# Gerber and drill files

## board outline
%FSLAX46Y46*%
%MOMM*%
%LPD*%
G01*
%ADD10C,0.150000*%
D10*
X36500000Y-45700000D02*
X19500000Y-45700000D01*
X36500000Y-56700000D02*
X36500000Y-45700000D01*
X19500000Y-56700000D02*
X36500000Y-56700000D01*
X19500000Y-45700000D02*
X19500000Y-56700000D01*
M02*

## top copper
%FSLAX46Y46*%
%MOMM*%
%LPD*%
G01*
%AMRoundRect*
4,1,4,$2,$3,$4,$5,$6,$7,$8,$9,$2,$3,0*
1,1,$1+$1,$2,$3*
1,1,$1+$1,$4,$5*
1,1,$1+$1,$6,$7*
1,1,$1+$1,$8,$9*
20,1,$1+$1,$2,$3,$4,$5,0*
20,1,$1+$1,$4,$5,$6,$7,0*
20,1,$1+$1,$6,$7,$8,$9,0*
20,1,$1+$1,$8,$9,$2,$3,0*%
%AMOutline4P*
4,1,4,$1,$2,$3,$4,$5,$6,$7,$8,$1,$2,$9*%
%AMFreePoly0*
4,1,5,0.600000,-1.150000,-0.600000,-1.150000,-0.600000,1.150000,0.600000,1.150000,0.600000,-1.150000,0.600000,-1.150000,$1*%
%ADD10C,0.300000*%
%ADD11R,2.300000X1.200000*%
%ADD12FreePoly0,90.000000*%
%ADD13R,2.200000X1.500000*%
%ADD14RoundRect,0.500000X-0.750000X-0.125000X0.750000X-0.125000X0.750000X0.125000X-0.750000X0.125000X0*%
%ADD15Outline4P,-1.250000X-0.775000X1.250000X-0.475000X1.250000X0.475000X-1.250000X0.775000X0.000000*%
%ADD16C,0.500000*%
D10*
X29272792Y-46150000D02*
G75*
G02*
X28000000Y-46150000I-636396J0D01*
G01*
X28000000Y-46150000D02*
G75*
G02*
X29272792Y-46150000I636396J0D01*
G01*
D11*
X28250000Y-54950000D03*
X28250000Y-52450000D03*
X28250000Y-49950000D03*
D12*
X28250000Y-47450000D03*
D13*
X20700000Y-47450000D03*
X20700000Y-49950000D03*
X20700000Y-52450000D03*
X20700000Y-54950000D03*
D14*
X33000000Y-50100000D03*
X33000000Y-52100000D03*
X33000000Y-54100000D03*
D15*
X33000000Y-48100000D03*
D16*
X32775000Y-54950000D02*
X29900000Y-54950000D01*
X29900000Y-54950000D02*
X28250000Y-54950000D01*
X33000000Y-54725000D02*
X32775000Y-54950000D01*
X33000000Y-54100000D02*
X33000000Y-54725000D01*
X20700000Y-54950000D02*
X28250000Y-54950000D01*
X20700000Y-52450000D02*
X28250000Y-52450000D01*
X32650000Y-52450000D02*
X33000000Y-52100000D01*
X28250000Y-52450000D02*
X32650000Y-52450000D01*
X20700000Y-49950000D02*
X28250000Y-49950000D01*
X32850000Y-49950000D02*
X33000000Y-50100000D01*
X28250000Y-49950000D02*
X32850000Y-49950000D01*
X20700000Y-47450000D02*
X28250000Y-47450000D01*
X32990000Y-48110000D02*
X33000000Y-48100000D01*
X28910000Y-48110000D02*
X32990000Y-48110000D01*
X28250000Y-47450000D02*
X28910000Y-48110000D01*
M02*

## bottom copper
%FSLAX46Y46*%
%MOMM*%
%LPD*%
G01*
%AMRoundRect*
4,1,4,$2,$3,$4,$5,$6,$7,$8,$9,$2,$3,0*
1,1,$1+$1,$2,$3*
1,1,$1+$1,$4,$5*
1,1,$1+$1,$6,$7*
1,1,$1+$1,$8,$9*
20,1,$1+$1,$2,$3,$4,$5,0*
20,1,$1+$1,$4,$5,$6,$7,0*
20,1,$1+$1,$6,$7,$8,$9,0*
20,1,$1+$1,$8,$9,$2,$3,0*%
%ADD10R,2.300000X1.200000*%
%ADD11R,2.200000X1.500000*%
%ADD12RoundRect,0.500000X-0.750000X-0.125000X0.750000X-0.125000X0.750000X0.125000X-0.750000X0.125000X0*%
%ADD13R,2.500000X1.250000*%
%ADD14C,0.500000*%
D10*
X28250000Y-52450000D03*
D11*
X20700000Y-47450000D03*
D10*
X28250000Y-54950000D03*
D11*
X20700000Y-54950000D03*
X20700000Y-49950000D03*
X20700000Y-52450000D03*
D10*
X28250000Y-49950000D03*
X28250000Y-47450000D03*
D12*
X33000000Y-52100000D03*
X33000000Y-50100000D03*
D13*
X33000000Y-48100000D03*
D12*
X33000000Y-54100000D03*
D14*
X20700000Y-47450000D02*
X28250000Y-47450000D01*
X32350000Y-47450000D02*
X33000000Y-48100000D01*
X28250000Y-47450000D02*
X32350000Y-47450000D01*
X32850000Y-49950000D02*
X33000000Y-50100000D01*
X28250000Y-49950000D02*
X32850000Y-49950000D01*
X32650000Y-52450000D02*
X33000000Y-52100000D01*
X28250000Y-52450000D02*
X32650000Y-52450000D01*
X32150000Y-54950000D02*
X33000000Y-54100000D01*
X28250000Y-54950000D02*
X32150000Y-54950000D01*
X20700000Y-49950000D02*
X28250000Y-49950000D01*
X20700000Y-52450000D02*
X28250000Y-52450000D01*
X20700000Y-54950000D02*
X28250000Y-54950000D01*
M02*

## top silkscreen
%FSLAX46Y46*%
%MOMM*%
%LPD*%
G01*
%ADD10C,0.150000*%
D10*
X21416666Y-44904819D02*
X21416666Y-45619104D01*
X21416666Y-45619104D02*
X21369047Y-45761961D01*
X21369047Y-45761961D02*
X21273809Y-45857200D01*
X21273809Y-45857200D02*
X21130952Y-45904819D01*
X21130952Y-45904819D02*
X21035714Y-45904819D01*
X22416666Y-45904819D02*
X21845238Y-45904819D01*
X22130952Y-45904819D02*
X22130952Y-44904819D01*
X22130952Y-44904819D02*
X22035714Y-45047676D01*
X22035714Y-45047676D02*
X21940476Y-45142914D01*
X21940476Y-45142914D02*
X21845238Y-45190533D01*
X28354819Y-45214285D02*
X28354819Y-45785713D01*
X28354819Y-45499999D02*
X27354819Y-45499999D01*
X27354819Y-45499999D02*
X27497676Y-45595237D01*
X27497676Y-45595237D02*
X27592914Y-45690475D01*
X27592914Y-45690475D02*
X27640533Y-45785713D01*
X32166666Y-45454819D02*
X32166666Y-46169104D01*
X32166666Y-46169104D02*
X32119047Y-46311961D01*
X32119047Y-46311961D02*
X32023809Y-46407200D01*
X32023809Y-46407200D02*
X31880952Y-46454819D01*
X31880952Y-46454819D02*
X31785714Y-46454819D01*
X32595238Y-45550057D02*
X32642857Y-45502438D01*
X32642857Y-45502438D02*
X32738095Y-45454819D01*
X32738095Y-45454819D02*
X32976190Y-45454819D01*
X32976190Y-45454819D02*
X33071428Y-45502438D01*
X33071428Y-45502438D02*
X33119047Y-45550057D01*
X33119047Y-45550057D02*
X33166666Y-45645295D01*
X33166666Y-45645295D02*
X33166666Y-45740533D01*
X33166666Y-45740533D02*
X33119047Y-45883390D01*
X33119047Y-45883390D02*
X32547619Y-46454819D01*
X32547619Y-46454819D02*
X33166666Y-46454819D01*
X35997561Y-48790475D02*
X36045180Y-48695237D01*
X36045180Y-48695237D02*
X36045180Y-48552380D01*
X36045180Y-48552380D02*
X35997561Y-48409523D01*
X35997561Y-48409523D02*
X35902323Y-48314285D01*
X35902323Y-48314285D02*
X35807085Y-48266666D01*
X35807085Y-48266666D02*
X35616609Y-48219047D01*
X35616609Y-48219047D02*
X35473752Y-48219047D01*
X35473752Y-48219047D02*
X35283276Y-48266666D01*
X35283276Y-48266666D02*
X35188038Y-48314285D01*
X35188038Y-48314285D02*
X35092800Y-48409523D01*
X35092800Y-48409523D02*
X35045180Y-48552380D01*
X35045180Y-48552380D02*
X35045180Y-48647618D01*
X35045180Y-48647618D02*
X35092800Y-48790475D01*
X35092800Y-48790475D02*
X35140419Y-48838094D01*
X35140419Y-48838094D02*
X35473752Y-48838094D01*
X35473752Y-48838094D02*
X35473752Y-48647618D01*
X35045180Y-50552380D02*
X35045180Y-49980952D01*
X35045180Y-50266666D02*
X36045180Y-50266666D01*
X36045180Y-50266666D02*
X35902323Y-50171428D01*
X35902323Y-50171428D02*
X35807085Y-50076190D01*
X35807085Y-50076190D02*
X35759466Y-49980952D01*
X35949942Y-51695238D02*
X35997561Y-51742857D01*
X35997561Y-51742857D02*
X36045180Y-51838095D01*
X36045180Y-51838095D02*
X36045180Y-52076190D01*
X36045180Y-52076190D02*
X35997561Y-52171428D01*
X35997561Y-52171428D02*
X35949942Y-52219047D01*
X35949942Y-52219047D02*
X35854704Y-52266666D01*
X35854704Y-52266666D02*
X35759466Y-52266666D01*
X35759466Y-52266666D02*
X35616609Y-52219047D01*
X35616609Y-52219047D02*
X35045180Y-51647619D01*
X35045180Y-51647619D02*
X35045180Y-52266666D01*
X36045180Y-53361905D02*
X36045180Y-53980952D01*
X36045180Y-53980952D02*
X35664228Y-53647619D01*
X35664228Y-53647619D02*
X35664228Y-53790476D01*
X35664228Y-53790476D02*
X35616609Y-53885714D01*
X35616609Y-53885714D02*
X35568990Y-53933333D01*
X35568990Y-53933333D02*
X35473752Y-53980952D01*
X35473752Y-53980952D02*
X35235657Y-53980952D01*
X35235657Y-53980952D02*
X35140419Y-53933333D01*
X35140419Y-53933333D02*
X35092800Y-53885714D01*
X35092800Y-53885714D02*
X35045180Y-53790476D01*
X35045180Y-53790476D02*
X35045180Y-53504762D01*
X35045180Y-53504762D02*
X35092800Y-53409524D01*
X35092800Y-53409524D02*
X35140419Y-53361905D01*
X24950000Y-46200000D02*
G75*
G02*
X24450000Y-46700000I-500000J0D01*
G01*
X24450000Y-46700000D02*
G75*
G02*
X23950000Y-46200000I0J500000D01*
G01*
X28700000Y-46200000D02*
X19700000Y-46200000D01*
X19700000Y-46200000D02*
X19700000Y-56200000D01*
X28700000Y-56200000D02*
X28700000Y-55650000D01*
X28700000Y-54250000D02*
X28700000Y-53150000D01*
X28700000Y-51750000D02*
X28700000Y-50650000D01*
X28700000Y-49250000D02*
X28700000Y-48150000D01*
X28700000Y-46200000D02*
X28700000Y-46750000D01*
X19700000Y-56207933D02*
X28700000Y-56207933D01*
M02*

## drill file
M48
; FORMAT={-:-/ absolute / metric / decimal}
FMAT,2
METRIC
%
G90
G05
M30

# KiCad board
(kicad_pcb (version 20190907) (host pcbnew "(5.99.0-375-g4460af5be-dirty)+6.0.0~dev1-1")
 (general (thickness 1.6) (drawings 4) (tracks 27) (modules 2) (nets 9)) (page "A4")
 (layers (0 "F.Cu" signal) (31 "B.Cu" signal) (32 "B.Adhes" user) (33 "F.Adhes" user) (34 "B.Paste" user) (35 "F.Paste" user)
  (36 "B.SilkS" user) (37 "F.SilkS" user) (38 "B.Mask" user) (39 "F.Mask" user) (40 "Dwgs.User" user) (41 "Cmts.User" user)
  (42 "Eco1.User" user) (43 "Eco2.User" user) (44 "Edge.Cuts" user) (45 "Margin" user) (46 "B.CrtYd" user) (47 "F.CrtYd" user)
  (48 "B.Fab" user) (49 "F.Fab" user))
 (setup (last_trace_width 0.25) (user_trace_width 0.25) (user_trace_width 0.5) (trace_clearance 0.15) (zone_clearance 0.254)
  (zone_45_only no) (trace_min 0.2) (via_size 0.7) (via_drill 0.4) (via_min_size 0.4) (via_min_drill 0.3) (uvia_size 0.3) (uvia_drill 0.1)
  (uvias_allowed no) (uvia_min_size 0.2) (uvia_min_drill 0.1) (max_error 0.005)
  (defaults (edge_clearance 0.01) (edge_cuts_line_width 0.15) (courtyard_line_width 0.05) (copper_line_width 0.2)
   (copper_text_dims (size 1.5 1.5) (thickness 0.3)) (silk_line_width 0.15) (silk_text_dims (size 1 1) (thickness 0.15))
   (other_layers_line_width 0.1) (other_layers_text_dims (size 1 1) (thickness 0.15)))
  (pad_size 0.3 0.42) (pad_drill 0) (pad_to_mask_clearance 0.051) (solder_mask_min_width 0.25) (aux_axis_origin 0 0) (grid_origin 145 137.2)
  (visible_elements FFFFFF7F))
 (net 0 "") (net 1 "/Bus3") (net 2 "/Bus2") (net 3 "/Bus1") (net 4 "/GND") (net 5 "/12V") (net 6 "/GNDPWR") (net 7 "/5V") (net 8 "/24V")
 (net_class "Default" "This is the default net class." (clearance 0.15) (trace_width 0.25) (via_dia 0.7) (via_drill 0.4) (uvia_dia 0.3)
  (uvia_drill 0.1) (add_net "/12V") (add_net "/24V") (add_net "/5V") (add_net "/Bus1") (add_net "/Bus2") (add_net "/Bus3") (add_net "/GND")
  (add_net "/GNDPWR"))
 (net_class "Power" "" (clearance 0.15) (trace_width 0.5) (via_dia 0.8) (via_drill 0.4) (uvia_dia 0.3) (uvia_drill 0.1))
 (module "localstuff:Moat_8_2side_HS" (layer "F.Cu") (at 24.5 56.2 -90)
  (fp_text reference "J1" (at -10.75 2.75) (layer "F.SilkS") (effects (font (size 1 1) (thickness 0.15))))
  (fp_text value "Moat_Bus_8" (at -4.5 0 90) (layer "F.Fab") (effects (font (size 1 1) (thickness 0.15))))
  (fp_arc (start -10 0.05) (end -10 -0.45) (angle 90) (layer "F.SilkS") (width 0.15))
  (fp_arc (start -10 0.05) (end -9.5 0.05) (angle 90) (layer "F.SilkS") (width 0.15))
  (fp_line (start -10 -4.2) (end -10 4.8) (layer "F.SilkS") (width 0.15))
  (fp_line (start -10 4.8) (end 0 4.8) (layer "F.SilkS") (width 0.15))
  (fp_line (start 0 -4.2) (end -0.55 -4.2) (layer "F.SilkS") (width 0.15))
  (fp_line (start -1.95 -4.2) (end -3.05 -4.2) (layer "F.SilkS") (width 0.15))
  (fp_line (start -4.45 -4.2) (end -5.55 -4.2) (layer "F.SilkS") (width 0.15))
  (fp_line (start -6.95 -4.2) (end -8.05 -4.2) (layer "F.SilkS") (width 0.15))
  (fp_line (start -10 -4.2) (end -9.45 -4.2) (layer "F.SilkS") (width 0.15))
  (fp_line (start 0.007933 4.8) (end 0.007933 -4.2) (layer "F.SilkS") (width 0.15))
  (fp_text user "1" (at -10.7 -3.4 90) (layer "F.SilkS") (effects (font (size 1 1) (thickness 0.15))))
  (fp_circle (center -10.05 -4.136396) (end -9.413604 -4.136396) (layer "F.Cu") (width 0.3))
  (pad "4" smd rect (at -1.25 -3.75 270) (size 1.2 2.3) (layers "F.Cu" "F.Paste" "F.Mask") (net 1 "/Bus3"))
  (pad "3" smd rect (at -3.75 -3.75 270) (size 1.2 2.3) (layers "F.Cu" "F.Paste" "F.Mask") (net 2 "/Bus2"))
  (pad "2" smd rect (at -6.25 -3.75 270) (size 1.2 2.3) (layers "F.Cu" "F.Paste" "F.Mask") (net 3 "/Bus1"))
  (pad "1" smd custom (at -8.75 -3.75 90) (size 1.2 2.3) (layers "F.Cu" "F.Paste" "F.Mask") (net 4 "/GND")
   (options (clearance outline) (anchor rect)) (primitives))
  (pad "1" smd rect (at -8.75 3.8 270) (size 1.5 2.2) (layers "F.Cu" "F.Paste" "F.Mask") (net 4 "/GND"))
  (pad "2" smd rect (at -6.25 3.8 270) (size 1.5 2.2) (layers "F.Cu" "F.Paste" "F.Mask") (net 3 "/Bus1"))
  (pad "3" smd rect (at -3.75 3.8 270) (size 1.5 2.2) (layers "F.Cu" "F.Paste" "F.Mask") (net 2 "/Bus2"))
  (pad "4" smd rect (at -1.25 3.8 270) (size 1.5 2.2) (layers "F.Cu" "F.Paste" "F.Mask") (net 1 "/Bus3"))
  (pad "6" smd rect (at -3.75 -3.75 90) (size 1.2 2.3) (layers "B.Cu" "B.Paste" "B.Mask") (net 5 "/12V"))
  (pad "8" smd rect (at -8.75 3.8 90) (size 1.5 2.2) (layers "B.Cu" "B.Paste" "B.Mask") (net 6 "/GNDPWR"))
  (pad "5" smd rect (at -1.25 -3.75 90) (size 1.2 2.3) (layers "B.Cu" "B.Paste" "B.Mask") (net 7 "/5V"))
  (pad "5" smd rect (at -1.25 3.8 90) (size 1.5 2.2) (layers "B.Cu" "B.Paste" "B.Mask") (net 7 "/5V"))
  (pad "7" smd rect (at -6.25 3.8 90) (size 1.5 2.2) (layers "B.Cu" "B.Paste" "B.Mask") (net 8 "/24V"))
  (pad "6" smd rect (at -3.75 3.8 90) (size 1.5 2.2) (layers "B.Cu" "B.Paste" "B.Mask") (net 5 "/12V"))
  (pad "7" smd rect (at -6.25 -3.75 90) (size 1.2 2.3) (layers "B.Cu" "B.Paste" "B.Mask") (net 8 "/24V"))
  (pad "8" smd rect (at -8.75 -3.75 90) (size 1.2 2.3) (layers "B.Cu" "B.Paste" "B.Mask") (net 6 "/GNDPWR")))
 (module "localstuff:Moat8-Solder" (layer "F.Cu") (at 33 46.6)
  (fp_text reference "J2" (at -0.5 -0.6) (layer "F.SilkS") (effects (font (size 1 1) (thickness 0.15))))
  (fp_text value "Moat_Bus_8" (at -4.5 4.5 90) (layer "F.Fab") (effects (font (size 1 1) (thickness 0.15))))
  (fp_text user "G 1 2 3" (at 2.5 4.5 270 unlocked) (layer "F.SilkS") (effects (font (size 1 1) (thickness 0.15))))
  (pad "6" smd roundrect (at 0 5.5) (size 2.5 1.25) (layers "B.Cu" "B.Mask") (roundrect_rratio 0.4) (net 5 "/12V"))
  (pad "7" smd roundrect (at 0 3.5) (size 2.5 1.25) (layers "B.Cu" "B.Mask") (roundrect_rratio 0.4) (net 8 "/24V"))
  (pad "8" smd rect (at 0 1.5) (size 2.5 1.25) (layers "B.Cu" "B.Mask") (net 6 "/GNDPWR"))
  (pad "5" smd roundrect (at 0 7.5) (size 2.5 1.25) (layers "B.Cu" "B.Mask") (roundrect_rratio 0.4) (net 7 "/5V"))
  (pad "2" smd roundrect (at 0 3.5) (size 2.5 1.25) (layers "F.Cu" "F.Mask") (roundrect_rratio 0.4) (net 3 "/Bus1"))
  (pad "3" smd roundrect (at 0 5.5) (size 2.5 1.25) (layers "F.Cu" "F.Mask") (roundrect_rratio 0.4) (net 2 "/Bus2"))
  (pad "4" smd roundrect (at 0 7.5) (size 2.5 1.25) (layers "F.Cu" "F.Mask") (roundrect_rratio 0.4) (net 1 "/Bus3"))
  (pad "1" smd trapezoid (at 0 1.5) (size 2.5 1.25) (rect_delta 0.3 0) (layers "F.Cu" "F.Mask") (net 4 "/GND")))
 (gr_line (start 36.5 45.7) (end 19.5 45.7) (layer "Edge.Cuts") (width 0.15))
 (gr_line (start 36.5 56.7) (end 36.5 45.7) (layer "Edge.Cuts") (width 0.15))
 (gr_line (start 19.5 56.7) (end 36.5 56.7) (layer "Edge.Cuts") (width 0.15))
 (gr_line (start 19.5 45.7) (end 19.5 56.7) (layer "Edge.Cuts") (width 0.15))
 (segment (start 32.775 54.95) (end 29.9 54.95) (width 0.5) (layer "F.Cu") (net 1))
 (segment (start 29.9 54.95) (end 28.25 54.95) (width 0.5) (layer "F.Cu") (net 1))
 (segment (start 33 54.725) (end 32.775 54.95) (width 0.5) (layer "F.Cu") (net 1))
 (segment (start 33 54.1) (end 33 54.725) (width 0.5) (layer "F.Cu") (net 1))
 (segment (start 20.7 54.95) (end 28.25 54.95) (width 0.5) (layer "F.Cu") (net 1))
 (segment (start 20.7 52.45) (end 28.25 52.45) (width 0.5) (layer "F.Cu") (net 2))
 (segment (start 32.65 52.45) (end 33 52.1) (width 0.5) (layer "F.Cu") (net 2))
 (segment (start 28.25 52.45) (end 32.65 52.45) (width 0.5) (layer "F.Cu") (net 2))
 (segment (start 20.7 49.95) (end 28.25 49.95) (width 0.5) (layer "F.Cu") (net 3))
 (segment (start 32.85 49.95) (end 33 50.1) (width 0.5) (layer "F.Cu") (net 3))
 (segment (start 28.25 49.95) (end 32.85 49.95) (width 0.5) (layer "F.Cu") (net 3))
 (segment (start 20.7 47.45) (end 28.25 47.45) (width 0.5) (layer "F.Cu") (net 4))
 (segment (start 32.99 48.11) (end 33 48.1) (width 0.5) (layer "F.Cu") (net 4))
 (segment (start 28.91 48.11) (end 32.99 48.11) (width 0.5) (layer "F.Cu") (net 4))
 (segment (start 28.25 47.45) (end 28.91 48.11) (width 0.5) (layer "F.Cu") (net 4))
 (segment (start 20.7 47.45) (end 28.25 47.45) (width 0.5) (layer "B.Cu") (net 6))
 (segment (start 32.35 47.45) (end 33 48.1) (width 0.5) (layer "B.Cu") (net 6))
 (segment (start 28.25 47.45) (end 32.35 47.45) (width 0.5) (layer "B.Cu") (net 6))
 (segment (start 32.85 49.95) (end 33 50.1) (width 0.5) (layer "B.Cu") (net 8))
 (segment (start 28.25 49.95) (end 32.85 49.95) (width 0.5) (layer "B.Cu") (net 8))
 (segment (start 32.65 52.45) (end 33 52.1) (width 0.5) (layer "B.Cu") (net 5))
 (segment (start 28.25 52.45) (end 32.65 52.45) (width 0.5) (layer "B.Cu") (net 5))
 (segment (start 32.15 54.95) (end 33 54.1) (width 0.5) (layer "B.Cu") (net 7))
 (segment (start 28.25 54.95) (end 32.15 54.95) (width 0.5) (layer "B.Cu") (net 7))
 (segment (start 20.7 49.95) (end 28.25 49.95) (width 0.5) (layer "B.Cu") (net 8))
 (segment (start 20.7 52.45) (end 28.25 52.45) (width 0.5) (layer "B.Cu") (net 5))
 (segment (start 20.7 54.95) (end 28.25 54.95) (width 0.5) (layer "B.Cu") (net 7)))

